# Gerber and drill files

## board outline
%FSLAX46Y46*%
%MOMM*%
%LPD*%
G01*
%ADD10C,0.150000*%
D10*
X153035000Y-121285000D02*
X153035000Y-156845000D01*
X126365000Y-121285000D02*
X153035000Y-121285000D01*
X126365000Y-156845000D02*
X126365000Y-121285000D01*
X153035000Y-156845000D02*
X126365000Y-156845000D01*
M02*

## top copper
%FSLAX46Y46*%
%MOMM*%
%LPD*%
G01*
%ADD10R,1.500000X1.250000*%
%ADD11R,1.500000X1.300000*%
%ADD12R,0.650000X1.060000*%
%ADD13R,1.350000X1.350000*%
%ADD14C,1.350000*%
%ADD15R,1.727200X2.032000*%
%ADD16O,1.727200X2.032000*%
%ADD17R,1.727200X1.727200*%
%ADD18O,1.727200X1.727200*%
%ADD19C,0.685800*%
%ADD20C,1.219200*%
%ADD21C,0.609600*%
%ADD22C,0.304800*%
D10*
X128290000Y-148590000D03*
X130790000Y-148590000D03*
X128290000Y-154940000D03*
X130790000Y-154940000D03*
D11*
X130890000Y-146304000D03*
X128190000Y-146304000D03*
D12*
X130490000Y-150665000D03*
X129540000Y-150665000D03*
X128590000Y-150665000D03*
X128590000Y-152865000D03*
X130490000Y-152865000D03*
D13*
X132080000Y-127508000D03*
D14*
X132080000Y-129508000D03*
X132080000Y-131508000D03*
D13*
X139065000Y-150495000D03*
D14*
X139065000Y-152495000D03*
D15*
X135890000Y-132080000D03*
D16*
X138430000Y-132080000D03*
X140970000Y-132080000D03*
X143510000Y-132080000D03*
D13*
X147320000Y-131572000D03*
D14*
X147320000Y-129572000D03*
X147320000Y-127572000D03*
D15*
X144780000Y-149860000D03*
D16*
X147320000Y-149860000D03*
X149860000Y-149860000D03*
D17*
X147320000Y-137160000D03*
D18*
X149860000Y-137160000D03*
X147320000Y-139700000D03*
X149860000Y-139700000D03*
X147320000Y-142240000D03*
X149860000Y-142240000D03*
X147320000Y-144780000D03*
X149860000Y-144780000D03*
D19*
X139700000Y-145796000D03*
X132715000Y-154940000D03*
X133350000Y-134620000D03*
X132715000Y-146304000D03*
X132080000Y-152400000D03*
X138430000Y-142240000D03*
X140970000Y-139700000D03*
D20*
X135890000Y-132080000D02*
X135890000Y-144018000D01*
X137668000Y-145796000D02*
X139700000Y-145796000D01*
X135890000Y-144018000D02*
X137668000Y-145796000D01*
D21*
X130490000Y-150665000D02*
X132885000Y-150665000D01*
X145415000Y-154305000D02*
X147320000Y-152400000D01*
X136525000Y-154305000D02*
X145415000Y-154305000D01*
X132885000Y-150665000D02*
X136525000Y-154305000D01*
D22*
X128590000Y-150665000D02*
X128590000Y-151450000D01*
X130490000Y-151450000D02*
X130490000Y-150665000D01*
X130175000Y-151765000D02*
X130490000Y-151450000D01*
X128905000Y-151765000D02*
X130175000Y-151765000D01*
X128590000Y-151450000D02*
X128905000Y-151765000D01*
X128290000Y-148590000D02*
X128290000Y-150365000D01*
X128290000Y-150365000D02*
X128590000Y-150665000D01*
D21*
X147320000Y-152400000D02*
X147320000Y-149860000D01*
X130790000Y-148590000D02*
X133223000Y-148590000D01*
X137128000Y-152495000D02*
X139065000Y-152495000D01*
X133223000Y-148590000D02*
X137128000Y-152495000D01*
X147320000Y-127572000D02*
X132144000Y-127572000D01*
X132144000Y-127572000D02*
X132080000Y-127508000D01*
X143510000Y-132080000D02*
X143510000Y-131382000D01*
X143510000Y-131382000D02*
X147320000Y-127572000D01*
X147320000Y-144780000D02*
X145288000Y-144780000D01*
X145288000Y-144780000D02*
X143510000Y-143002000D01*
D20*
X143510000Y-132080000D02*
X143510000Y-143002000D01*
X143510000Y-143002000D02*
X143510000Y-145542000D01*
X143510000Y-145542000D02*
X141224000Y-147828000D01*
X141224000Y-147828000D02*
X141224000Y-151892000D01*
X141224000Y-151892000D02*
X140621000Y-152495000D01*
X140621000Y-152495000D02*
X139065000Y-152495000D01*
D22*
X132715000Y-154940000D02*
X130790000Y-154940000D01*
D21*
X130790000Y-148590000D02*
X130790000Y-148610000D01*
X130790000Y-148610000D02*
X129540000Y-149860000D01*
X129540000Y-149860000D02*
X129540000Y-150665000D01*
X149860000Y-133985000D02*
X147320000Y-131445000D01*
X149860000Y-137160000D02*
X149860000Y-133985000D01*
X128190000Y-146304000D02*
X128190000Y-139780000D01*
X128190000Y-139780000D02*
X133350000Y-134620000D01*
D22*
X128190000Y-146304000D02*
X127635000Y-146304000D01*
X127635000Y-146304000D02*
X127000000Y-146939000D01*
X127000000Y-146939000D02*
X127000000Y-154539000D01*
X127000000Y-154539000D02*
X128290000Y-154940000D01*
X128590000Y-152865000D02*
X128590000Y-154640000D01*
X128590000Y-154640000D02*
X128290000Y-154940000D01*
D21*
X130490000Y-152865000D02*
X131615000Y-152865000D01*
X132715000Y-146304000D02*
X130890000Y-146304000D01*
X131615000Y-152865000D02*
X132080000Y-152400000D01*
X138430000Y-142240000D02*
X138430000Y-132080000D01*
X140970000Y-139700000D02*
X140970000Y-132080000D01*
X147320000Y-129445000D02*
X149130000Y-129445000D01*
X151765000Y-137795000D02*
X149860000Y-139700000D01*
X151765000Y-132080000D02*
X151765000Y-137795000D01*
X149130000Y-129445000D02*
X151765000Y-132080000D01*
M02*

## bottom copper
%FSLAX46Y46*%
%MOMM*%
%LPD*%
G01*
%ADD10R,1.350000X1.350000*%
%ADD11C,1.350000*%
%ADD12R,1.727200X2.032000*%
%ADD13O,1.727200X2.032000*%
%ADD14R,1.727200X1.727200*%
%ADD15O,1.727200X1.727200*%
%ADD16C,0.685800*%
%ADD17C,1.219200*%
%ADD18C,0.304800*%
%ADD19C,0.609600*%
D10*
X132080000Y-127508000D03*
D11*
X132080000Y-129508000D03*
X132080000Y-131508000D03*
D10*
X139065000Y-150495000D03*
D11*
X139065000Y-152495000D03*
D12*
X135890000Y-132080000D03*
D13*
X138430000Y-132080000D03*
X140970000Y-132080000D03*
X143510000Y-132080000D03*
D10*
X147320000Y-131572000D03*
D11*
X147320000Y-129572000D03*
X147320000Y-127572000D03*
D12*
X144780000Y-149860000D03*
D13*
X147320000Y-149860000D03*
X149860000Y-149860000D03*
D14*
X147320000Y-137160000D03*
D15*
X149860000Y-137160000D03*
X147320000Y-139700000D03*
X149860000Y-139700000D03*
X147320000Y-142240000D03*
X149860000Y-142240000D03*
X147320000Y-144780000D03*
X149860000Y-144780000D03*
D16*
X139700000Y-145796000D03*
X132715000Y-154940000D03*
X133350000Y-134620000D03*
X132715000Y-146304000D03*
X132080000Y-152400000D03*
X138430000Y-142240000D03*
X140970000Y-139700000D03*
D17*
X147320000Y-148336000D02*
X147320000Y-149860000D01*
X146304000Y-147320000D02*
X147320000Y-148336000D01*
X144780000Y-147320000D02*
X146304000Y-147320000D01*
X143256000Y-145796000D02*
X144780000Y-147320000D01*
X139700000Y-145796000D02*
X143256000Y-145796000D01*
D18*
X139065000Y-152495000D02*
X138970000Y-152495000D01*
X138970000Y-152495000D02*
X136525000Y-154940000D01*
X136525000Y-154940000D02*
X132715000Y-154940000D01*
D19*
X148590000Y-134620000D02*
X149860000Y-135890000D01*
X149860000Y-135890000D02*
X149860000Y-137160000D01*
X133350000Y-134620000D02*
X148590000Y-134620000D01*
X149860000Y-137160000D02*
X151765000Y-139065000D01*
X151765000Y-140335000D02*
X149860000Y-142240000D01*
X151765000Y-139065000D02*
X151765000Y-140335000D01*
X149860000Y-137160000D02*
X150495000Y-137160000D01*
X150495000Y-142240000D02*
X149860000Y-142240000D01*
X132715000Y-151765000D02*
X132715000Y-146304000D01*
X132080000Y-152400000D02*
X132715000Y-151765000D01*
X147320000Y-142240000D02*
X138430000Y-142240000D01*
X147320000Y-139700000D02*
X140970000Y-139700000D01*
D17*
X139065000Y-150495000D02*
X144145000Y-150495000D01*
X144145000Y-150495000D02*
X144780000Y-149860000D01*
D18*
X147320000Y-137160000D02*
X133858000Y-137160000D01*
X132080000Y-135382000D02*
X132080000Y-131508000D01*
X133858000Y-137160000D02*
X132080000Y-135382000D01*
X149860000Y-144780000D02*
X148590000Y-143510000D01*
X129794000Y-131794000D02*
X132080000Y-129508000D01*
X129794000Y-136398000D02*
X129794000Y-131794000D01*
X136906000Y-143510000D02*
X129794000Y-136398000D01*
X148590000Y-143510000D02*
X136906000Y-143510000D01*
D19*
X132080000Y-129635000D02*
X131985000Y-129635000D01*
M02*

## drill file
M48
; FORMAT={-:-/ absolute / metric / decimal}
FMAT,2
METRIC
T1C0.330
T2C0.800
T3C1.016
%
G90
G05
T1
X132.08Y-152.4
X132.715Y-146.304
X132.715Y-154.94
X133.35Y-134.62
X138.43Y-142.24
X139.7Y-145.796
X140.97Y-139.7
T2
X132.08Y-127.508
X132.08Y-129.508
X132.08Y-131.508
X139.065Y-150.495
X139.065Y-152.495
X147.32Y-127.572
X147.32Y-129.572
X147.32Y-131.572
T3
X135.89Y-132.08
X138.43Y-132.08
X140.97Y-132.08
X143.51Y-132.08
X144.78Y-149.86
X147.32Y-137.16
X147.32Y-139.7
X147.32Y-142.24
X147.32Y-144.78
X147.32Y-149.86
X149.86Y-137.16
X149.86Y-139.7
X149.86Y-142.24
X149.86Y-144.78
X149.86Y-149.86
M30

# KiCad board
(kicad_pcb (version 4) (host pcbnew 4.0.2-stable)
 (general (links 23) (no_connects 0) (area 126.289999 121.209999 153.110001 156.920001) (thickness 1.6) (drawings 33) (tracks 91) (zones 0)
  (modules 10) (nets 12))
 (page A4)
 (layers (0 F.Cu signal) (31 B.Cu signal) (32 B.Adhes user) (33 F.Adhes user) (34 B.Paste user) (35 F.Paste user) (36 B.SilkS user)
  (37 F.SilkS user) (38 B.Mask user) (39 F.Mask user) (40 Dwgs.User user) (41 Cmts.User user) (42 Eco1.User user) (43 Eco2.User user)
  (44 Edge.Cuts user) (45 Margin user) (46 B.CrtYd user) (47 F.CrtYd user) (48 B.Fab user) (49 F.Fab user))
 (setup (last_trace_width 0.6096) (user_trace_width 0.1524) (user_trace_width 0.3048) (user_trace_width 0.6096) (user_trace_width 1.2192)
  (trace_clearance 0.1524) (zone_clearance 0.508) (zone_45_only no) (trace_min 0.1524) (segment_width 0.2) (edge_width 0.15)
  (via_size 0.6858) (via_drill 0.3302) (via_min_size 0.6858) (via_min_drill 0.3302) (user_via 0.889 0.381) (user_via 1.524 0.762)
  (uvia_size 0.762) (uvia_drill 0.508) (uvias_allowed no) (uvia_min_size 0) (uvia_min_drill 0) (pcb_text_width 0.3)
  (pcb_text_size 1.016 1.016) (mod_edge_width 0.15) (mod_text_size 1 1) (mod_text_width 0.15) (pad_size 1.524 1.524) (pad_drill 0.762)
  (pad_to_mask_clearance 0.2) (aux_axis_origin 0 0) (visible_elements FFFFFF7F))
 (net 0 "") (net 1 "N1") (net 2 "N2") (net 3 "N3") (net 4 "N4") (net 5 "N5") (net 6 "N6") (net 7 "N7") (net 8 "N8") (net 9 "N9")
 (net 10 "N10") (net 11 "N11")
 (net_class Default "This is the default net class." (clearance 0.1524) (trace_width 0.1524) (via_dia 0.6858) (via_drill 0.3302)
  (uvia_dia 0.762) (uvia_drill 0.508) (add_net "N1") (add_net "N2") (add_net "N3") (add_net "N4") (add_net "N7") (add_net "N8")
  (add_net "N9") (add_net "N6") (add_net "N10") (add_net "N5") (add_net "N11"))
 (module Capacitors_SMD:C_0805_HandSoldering (layer F.Cu) (at 129.54 148.59)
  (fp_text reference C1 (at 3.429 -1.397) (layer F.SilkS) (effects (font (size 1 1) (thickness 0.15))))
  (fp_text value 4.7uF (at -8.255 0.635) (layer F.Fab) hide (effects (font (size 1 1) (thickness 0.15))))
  (pad 1 smd rect (at -1.25 0) (size 1.5 1.25) (layers F.Cu F.Paste F.Mask) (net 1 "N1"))
  (pad 2 smd rect (at 1.25 0) (size 1.5 1.25) (layers F.Cu F.Paste F.Mask) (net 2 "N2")))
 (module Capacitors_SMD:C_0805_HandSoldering (layer F.Cu) (at 129.54 154.94)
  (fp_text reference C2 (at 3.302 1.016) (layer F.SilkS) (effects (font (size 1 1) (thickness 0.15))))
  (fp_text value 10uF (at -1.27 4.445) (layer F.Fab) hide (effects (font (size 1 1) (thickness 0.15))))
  (pad 1 smd rect (at -1.25 0) (size 1.5 1.25) (layers F.Cu F.Paste F.Mask) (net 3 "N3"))
  (pad 2 smd rect (at 1.25 0) (size 1.5 1.25) (layers F.Cu F.Paste F.Mask) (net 2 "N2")))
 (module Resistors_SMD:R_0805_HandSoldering (layer F.Cu) (at 129.54 146.304 180)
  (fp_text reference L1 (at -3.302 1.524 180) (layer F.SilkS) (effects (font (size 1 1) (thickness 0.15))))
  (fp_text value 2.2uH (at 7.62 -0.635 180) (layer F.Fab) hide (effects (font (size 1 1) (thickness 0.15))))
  (pad 1 smd rect (at -1.35 0 180) (size 1.5 1.3) (layers F.Cu F.Paste F.Mask) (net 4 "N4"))
  (pad 2 smd rect (at 1.35 0 180) (size 1.5 1.3) (layers F.Cu F.Paste F.Mask) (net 3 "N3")))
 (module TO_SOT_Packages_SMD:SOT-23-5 (layer F.Cu) (at 129.54 151.765 270)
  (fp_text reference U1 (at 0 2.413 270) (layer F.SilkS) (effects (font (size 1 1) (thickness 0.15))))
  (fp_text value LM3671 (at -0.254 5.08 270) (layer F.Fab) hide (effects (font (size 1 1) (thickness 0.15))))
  (pad 1 smd rect (at -1.1 -0.95 270) (size 1.06 0.65) (layers F.Cu F.Paste F.Mask) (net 1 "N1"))
  (pad 2 smd rect (at -1.1 0 270) (size 1.06 0.65) (layers F.Cu F.Paste F.Mask) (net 2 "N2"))
  (pad 3 smd rect (at -1.1 0.95 270) (size 1.06 0.65) (layers F.Cu F.Paste F.Mask) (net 1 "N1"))
  (pad 4 smd rect (at 1.1 0.95 270) (size 1.06 0.65) (layers F.Cu F.Paste F.Mask) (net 3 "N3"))
  (pad 5 smd rect (at 1.1 -0.95 270) (size 1.06 0.65) (layers F.Cu F.Paste F.Mask) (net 4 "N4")))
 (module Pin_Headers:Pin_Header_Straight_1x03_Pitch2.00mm (layer F.Cu) (at 132.08 127.508)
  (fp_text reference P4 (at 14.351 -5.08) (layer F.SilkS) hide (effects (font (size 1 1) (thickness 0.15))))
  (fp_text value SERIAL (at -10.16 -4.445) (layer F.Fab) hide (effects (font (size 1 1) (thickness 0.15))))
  (pad 1 thru_hole rect (at 0 0) (size 1.35 1.35) (drill 0.8) (layers *.Cu *.Mask) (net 2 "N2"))
  (pad 2 thru_hole circle (at 0 2) (size 1.35 1.35) (drill 0.8) (layers *.Cu *.Mask) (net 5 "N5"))
  (pad 3 thru_hole circle (at 0 4) (size 1.35 1.35) (drill 0.8) (layers *.Cu *.Mask) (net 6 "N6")))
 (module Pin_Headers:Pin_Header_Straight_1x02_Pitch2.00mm (layer F.Cu) (at 139.065 150.495)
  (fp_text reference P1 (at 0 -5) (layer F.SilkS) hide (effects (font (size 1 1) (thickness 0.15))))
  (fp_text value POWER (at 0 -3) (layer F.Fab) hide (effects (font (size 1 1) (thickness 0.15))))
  (pad 1 thru_hole rect (at 0 0) (size 1.35 1.35) (drill 0.8) (layers *.Cu *.Mask) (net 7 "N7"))
  (pad 2 thru_hole circle (at 0 2) (size 1.35 1.35) (drill 0.8) (layers *.Cu *.Mask) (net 2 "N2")))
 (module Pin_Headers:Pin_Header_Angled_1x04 (layer F.Cu) (at 135.89 132.08 90)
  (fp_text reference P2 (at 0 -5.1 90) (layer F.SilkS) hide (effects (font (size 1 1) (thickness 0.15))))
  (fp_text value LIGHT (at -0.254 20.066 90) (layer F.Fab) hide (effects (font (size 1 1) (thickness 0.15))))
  (pad 1 thru_hole rect (at 0 0 90) (size 2.032 1.7272) (drill 1.016) (layers *.Cu *.Mask) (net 1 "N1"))
  (pad 2 thru_hole oval (at 0 2.54 90) (size 2.032 1.7272) (drill 1.016) (layers *.Cu *.Mask) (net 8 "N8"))
  (pad 3 thru_hole oval (at 0 5.08 90) (size 2.032 1.7272) (drill 1.016) (layers *.Cu *.Mask) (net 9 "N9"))
  (pad 4 thru_hole oval (at 0 7.62 90) (size 2.032 1.7272) (drill 1.016) (layers *.Cu *.Mask) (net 2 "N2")))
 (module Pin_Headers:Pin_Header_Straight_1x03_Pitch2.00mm (layer F.Cu) (at 147.32 131.572 180)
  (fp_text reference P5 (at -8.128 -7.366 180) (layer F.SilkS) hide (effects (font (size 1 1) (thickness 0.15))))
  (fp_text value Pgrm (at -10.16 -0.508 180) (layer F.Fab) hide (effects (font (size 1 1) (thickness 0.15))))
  (pad 1 thru_hole rect (at 0 0 180) (size 1.35 1.35) (drill 0.8) (layers *.Cu *.Mask) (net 3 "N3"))
  (pad 2 thru_hole circle (at 0 2 180) (size 1.35 1.35) (drill 0.8) (layers *.Cu *.Mask) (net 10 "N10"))
  (pad 3 thru_hole circle (at 0 4 180) (size 1.35 1.35) (drill 0.8) (layers *.Cu *.Mask) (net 2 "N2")))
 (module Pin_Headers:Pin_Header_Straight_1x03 (layer F.Cu) (at 144.78 149.86 90)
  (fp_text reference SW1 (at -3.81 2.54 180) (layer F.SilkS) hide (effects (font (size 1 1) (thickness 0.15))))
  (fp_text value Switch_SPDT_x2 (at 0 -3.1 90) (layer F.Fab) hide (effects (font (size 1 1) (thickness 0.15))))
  (pad 1 thru_hole rect (at 0 0 90) (size 2.032 1.7272) (drill 1.016) (layers *.Cu *.Mask) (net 7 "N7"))
  (pad 2 thru_hole oval (at 0 2.54 90) (size 2.032 1.7272) (drill 1.016) (layers *.Cu *.Mask) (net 1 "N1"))
  (pad 3 thru_hole oval (at 0 5.08 90) (size 2.032 1.7272) (drill 1.016) (layers *.Cu *.Mask) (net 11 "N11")))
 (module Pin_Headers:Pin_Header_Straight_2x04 (layer F.Cu) (at 147.32 137.16)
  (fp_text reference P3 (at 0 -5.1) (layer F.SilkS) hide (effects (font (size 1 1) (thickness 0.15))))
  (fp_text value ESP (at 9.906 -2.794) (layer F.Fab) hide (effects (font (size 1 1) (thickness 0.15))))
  (pad 1 thru_hole rect (at 0 0) (size 1.7272 1.7272) (drill 1.016) (layers *.Cu *.Mask) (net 6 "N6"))
  (pad 2 thru_hole oval (at 2.54 0) (size 1.7272 1.7272) (drill 1.016) (layers *.Cu *.Mask) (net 3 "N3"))
  (pad 3 thru_hole oval (at 0 2.54) (size 1.7272 1.7272) (drill 1.016) (layers *.Cu *.Mask) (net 9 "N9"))
  (pad 4 thru_hole oval (at 2.54 2.54) (size 1.7272 1.7272) (drill 1.016) (layers *.Cu *.Mask) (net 10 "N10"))
  (pad 5 thru_hole oval (at 0 5.08) (size 1.7272 1.7272) (drill 1.016) (layers *.Cu *.Mask) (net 8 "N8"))
  (pad 6 thru_hole oval (at 2.54 5.08) (size 1.7272 1.7272) (drill 1.016) (layers *.Cu *.Mask) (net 3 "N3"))
  (pad 7 thru_hole oval (at 0 7.62) (size 1.7272 1.7272) (drill 1.016) (layers *.Cu *.Mask) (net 2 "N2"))
  (pad 8 thru_hole oval (at 2.54 7.62) (size 1.7272 1.7272) (drill 1.016) (layers *.Cu *.Mask) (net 5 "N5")))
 (gr_line (start 153.035 121.285) (end 153.035 156.845) (angle 90) (layer Edge.Cuts) (width 0.15))
 (gr_line (start 126.365 121.285) (end 153.035 121.285) (angle 90) (layer Edge.Cuts) (width 0.15))
 (gr_line (start 126.365 156.845) (end 126.365 121.285) (angle 90) (layer Edge.Cuts) (width 0.15))
 (gr_line (start 153.035 156.845) (end 126.365 156.845) (angle 90) (layer Edge.Cuts) (width 0.15))
 (segment (start 135.89 132.08) (end 135.89 144.018) (width 1.2192) (layer F.Cu) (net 1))
 (segment (start 147.32 148.336) (end 147.32 149.86) (width 1.2192) (layer B.Cu) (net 1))
 (segment (start 146.304 147.32) (end 147.32 148.336) (width 1.2192) (layer B.Cu) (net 1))
 (segment (start 144.78 147.32) (end 146.304 147.32) (width 1.2192) (layer B.Cu) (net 1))
 (segment (start 143.256 145.796) (end 144.78 147.32) (width 1.2192) (layer B.Cu) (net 1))
 (segment (start 139.7 145.796) (end 143.256 145.796) (width 1.2192) (layer B.Cu) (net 1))
 (via (at 139.7 145.796) (size 0.6858) (drill 0.3302) (layers F.Cu B.Cu) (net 1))
 (segment (start 137.668 145.796) (end 139.7 145.796) (width 1.2192) (layer F.Cu) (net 1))
 (segment (start 135.89 144.018) (end 137.668 145.796) (width 1.2192) (layer F.Cu) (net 1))
 (segment (start 130.49 150.665) (end 132.885 150.665) (width 0.6096) (layer F.Cu) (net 1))
 (segment (start 145.415 154.305) (end 147.32 152.4) (width 0.6096) (layer F.Cu) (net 1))
 (segment (start 136.525 154.305) (end 145.415 154.305) (width 0.6096) (layer F.Cu) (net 1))
 (segment (start 132.885 150.665) (end 136.525 154.305) (width 0.6096) (layer F.Cu) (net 1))
 (segment (start 128.59 150.665) (end 128.59 151.45) (width 0.3048) (layer F.Cu) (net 1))
 (segment (start 130.49 151.45) (end 130.49 150.665) (width 0.3048) (layer F.Cu) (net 1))
 (segment (start 130.175 151.765) (end 130.49 151.45) (width 0.3048) (layer F.Cu) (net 1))
 (segment (start 128.905 151.765) (end 130.175 151.765) (width 0.3048) (layer F.Cu) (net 1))
 (segment (start 128.59 151.45) (end 128.905 151.765) (width 0.3048) (layer F.Cu) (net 1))
 (segment (start 128.29 148.59) (end 128.29 150.365) (width 0.3048) (layer F.Cu) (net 1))
 (segment (start 128.29 150.365) (end 128.59 150.665) (width 0.3048) (layer F.Cu) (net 1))
 (segment (start 147.32 152.4) (end 147.32 149.86) (width 0.6096) (layer F.Cu) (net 1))
 (segment (start 130.79 148.59) (end 133.223 148.59) (width 0.6096) (layer F.Cu) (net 2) (status 400000))
 (segment (start 137.128 152.495) (end 139.065 152.495) (width 0.6096) (layer F.Cu) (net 2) (status 800000))
 (segment (start 133.223 148.59) (end 137.128 152.495) (width 0.6096) (layer F.Cu) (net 2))
 (segment (start 147.32 127.572) (end 132.144 127.572) (width 0.6096) (layer F.Cu) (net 2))
 (segment (start 132.144 127.572) (end 132.08 127.508) (width 0.6096) (layer F.Cu) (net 2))
 (segment (start 143.51 132.08) (end 143.51 131.382) (width 0.6096) (layer F.Cu) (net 2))
 (segment (start 143.51 131.382) (end 147.32 127.572) (width 0.6096) (layer F.Cu) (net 2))
 (segment (start 147.32 144.78) (end 145.288 144.78) (width 0.6096) (layer F.Cu) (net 2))
 (segment (start 145.288 144.78) (end 143.51 143.002) (width 0.6096) (layer F.Cu) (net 2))
 (segment (start 143.51 132.08) (end 143.51 143.002) (width 1.2192) (layer F.Cu) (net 2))
 (segment (start 143.51 143.002) (end 143.51 145.542) (width 1.2192) (layer F.Cu) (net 2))
 (segment (start 143.51 145.542) (end 141.224 147.828) (width 1.2192) (layer F.Cu) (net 2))
 (segment (start 141.224 147.828) (end 141.224 151.892) (width 1.2192) (layer F.Cu) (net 2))
 (segment (start 141.224 151.892) (end 140.621 152.495) (width 1.2192) (layer F.Cu) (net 2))
 (segment (start 140.621 152.495) (end 139.065 152.495) (width 1.2192) (layer F.Cu) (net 2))
 (segment (start 139.065 152.495) (end 138.97 152.495) (width 0.3048) (layer B.Cu) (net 2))
 (segment (start 138.97 152.495) (end 136.525 154.94) (width 0.3048) (layer B.Cu) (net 2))
 (segment (start 132.715 154.94) (end 130.79 154.94) (width 0.3048) (layer F.Cu) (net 2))
 (via (at 132.715 154.94) (size 0.6858) (drill 0.3302) (layers F.Cu B.Cu) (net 2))
 (segment (start 136.525 154.94) (end 132.715 154.94) (width 0.3048) (layer B.Cu) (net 2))
 (segment (start 130.79 148.59) (end 130.79 148.61) (width 0.6096) (layer F.Cu) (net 2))
 (segment (start 130.79 148.61) (end 129.54 149.86) (width 0.6096) (layer F.Cu) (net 2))
 (segment (start 129.54 149.86) (end 129.54 150.665) (width 0.6096) (layer F.Cu) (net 2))
 (segment (start 149.86 133.985) (end 147.32 131.445) (width 0.6096) (layer F.Cu) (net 3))
 (segment (start 149.86 137.16) (end 149.86 133.985) (width 0.6096) (layer F.Cu) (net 3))
 (segment (start 148.59 134.62) (end 149.86 135.89) (width 0.6096) (layer B.Cu) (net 3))
 (segment (start 149.86 135.89) (end 149.86 137.16) (width 0.6096) (layer B.Cu) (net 3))
 (segment (start 133.35 134.62) (end 148.59 134.62) (width 0.6096) (layer B.Cu) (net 3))
 (segment (start 149.86 137.16) (end 151.765 139.065) (width 0.6096) (layer B.Cu) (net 3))
 (segment (start 151.765 140.335) (end 149.86 142.24) (width 0.6096) (layer B.Cu) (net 3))
 (segment (start 151.765 139.065) (end 151.765 140.335) (width 0.6096) (layer B.Cu) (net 3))
 (segment (start 149.86 137.16) (end 150.495 137.16) (width 0.6096) (layer B.Cu) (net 3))
 (segment (start 150.495 142.24) (end 149.86 142.24) (width 0.6096) (layer B.Cu) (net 3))
 (segment (start 128.19 146.304) (end 128.19 139.78) (width 0.6096) (layer F.Cu) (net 3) (status 10))
 (segment (start 128.19 139.78) (end 133.35 134.62) (width 0.6096) (layer F.Cu) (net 3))
 (via (at 133.35 134.62) (size 0.6858) (drill 0.3302) (layers F.Cu B.Cu) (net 3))
 (segment (start 128.19 146.304) (end 127.635 146.304) (width 0.3048) (layer F.Cu) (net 3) (status 30))
 (segment (start 127.635 146.304) (end 127 146.939) (width 0.3048) (layer F.Cu) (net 3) (status 10))
 (segment (start 127 146.939) (end 127 154.539) (width 0.3048) (layer F.Cu) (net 3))
 (segment (start 127 154.539) (end 128.29 154.94) (width 0.3048) (layer F.Cu) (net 3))
 (segment (start 128.59 152.865) (end 128.59 154.64) (width 0.3048) (layer F.Cu) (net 3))
 (segment (start 128.59 154.64) (end 128.29 154.94) (width 0.3048) (layer F.Cu) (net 3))
 (segment (start 130.49 152.865) (end 131.615 152.865) (width 0.6096) (layer F.Cu) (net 4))
 (segment (start 132.715 146.304) (end 130.89 146.304) (width 0.6096) (layer F.Cu) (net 4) (status 20))
 (via (at 132.715 146.304) (size 0.6858) (drill 0.3302) (layers F.Cu B.Cu) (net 4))
 (segment (start 132.715 151.765) (end 132.715 146.304) (width 0.6096) (layer B.Cu) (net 4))
 (segment (start 132.08 152.4) (end 132.715 151.765) (width 0.6096) (layer B.Cu) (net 4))
 (via (at 132.08 152.4) (size 0.6858) (drill 0.3302) (layers F.Cu B.Cu) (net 4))
 (segment (start 131.615 152.865) (end 132.08 152.4) (width 0.6096) (layer F.Cu) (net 4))
 (segment (start 147.32 142.24) (end 138.43 142.24) (width 0.6096) (layer B.Cu) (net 8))
 (segment (start 138.43 142.24) (end 138.43 132.08) (width 0.6096) (layer F.Cu) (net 8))
 (via (at 138.43 142.24) (size 0.6858) (drill 0.3302) (layers F.Cu B.Cu) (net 8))
 (segment (start 147.32 139.7) (end 140.97 139.7) (width 0.6096) (layer B.Cu) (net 9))
 (segment (start 140.97 139.7) (end 140.97 132.08) (width 0.6096) (layer F.Cu) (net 9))
 (via (at 140.97 139.7) (size 0.6858) (drill 0.3302) (layers F.Cu B.Cu) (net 9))
 (segment (start 139.065 150.495) (end 144.145 150.495) (width 1.2192) (layer B.Cu) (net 7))
 (segment (start 144.145 150.495) (end 144.78 149.86) (width 1.2192) (layer B.Cu) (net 7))
 (segment (start 147.32 137.16) (end 133.858 137.16) (width 0.3048) (layer B.Cu) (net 6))
 (segment (start 132.08 135.382) (end 132.08 131.508) (width 0.3048) (layer B.Cu) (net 6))
 (segment (start 133.858 137.16) (end 132.08 135.382) (width 0.3048) (layer B.Cu) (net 6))
 (segment (start 147.32 129.445) (end 149.13 129.445) (width 0.6096) (layer F.Cu) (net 10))
 (segment (start 151.765 137.795) (end 149.86 139.7) (width 0.6096) (layer F.Cu) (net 10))
 (segment (start 151.765 132.08) (end 151.765 137.795) (width 0.6096) (layer F.Cu) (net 10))
 (segment (start 149.13 129.445) (end 151.765 132.08) (width 0.6096) (layer F.Cu) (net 10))
 (segment (start 149.86 144.78) (end 148.59 143.51) (width 0.3048) (layer B.Cu) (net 5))
 (segment (start 129.794 131.794) (end 132.08 129.508) (width 0.3048) (layer B.Cu) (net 5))
 (segment (start 129.794 136.398) (end 129.794 131.794) (width 0.3048) (layer B.Cu) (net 5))
 (segment (start 136.906 143.51) (end 129.794 136.398) (width 0.3048) (layer B.Cu) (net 5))
 (segment (start 148.59 143.51) (end 136.906 143.51) (width 0.3048) (layer B.Cu) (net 5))
 (segment (start 132.08 129.635) (end 131.985 129.635) (width 0.6096) (layer B.Cu) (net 5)))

